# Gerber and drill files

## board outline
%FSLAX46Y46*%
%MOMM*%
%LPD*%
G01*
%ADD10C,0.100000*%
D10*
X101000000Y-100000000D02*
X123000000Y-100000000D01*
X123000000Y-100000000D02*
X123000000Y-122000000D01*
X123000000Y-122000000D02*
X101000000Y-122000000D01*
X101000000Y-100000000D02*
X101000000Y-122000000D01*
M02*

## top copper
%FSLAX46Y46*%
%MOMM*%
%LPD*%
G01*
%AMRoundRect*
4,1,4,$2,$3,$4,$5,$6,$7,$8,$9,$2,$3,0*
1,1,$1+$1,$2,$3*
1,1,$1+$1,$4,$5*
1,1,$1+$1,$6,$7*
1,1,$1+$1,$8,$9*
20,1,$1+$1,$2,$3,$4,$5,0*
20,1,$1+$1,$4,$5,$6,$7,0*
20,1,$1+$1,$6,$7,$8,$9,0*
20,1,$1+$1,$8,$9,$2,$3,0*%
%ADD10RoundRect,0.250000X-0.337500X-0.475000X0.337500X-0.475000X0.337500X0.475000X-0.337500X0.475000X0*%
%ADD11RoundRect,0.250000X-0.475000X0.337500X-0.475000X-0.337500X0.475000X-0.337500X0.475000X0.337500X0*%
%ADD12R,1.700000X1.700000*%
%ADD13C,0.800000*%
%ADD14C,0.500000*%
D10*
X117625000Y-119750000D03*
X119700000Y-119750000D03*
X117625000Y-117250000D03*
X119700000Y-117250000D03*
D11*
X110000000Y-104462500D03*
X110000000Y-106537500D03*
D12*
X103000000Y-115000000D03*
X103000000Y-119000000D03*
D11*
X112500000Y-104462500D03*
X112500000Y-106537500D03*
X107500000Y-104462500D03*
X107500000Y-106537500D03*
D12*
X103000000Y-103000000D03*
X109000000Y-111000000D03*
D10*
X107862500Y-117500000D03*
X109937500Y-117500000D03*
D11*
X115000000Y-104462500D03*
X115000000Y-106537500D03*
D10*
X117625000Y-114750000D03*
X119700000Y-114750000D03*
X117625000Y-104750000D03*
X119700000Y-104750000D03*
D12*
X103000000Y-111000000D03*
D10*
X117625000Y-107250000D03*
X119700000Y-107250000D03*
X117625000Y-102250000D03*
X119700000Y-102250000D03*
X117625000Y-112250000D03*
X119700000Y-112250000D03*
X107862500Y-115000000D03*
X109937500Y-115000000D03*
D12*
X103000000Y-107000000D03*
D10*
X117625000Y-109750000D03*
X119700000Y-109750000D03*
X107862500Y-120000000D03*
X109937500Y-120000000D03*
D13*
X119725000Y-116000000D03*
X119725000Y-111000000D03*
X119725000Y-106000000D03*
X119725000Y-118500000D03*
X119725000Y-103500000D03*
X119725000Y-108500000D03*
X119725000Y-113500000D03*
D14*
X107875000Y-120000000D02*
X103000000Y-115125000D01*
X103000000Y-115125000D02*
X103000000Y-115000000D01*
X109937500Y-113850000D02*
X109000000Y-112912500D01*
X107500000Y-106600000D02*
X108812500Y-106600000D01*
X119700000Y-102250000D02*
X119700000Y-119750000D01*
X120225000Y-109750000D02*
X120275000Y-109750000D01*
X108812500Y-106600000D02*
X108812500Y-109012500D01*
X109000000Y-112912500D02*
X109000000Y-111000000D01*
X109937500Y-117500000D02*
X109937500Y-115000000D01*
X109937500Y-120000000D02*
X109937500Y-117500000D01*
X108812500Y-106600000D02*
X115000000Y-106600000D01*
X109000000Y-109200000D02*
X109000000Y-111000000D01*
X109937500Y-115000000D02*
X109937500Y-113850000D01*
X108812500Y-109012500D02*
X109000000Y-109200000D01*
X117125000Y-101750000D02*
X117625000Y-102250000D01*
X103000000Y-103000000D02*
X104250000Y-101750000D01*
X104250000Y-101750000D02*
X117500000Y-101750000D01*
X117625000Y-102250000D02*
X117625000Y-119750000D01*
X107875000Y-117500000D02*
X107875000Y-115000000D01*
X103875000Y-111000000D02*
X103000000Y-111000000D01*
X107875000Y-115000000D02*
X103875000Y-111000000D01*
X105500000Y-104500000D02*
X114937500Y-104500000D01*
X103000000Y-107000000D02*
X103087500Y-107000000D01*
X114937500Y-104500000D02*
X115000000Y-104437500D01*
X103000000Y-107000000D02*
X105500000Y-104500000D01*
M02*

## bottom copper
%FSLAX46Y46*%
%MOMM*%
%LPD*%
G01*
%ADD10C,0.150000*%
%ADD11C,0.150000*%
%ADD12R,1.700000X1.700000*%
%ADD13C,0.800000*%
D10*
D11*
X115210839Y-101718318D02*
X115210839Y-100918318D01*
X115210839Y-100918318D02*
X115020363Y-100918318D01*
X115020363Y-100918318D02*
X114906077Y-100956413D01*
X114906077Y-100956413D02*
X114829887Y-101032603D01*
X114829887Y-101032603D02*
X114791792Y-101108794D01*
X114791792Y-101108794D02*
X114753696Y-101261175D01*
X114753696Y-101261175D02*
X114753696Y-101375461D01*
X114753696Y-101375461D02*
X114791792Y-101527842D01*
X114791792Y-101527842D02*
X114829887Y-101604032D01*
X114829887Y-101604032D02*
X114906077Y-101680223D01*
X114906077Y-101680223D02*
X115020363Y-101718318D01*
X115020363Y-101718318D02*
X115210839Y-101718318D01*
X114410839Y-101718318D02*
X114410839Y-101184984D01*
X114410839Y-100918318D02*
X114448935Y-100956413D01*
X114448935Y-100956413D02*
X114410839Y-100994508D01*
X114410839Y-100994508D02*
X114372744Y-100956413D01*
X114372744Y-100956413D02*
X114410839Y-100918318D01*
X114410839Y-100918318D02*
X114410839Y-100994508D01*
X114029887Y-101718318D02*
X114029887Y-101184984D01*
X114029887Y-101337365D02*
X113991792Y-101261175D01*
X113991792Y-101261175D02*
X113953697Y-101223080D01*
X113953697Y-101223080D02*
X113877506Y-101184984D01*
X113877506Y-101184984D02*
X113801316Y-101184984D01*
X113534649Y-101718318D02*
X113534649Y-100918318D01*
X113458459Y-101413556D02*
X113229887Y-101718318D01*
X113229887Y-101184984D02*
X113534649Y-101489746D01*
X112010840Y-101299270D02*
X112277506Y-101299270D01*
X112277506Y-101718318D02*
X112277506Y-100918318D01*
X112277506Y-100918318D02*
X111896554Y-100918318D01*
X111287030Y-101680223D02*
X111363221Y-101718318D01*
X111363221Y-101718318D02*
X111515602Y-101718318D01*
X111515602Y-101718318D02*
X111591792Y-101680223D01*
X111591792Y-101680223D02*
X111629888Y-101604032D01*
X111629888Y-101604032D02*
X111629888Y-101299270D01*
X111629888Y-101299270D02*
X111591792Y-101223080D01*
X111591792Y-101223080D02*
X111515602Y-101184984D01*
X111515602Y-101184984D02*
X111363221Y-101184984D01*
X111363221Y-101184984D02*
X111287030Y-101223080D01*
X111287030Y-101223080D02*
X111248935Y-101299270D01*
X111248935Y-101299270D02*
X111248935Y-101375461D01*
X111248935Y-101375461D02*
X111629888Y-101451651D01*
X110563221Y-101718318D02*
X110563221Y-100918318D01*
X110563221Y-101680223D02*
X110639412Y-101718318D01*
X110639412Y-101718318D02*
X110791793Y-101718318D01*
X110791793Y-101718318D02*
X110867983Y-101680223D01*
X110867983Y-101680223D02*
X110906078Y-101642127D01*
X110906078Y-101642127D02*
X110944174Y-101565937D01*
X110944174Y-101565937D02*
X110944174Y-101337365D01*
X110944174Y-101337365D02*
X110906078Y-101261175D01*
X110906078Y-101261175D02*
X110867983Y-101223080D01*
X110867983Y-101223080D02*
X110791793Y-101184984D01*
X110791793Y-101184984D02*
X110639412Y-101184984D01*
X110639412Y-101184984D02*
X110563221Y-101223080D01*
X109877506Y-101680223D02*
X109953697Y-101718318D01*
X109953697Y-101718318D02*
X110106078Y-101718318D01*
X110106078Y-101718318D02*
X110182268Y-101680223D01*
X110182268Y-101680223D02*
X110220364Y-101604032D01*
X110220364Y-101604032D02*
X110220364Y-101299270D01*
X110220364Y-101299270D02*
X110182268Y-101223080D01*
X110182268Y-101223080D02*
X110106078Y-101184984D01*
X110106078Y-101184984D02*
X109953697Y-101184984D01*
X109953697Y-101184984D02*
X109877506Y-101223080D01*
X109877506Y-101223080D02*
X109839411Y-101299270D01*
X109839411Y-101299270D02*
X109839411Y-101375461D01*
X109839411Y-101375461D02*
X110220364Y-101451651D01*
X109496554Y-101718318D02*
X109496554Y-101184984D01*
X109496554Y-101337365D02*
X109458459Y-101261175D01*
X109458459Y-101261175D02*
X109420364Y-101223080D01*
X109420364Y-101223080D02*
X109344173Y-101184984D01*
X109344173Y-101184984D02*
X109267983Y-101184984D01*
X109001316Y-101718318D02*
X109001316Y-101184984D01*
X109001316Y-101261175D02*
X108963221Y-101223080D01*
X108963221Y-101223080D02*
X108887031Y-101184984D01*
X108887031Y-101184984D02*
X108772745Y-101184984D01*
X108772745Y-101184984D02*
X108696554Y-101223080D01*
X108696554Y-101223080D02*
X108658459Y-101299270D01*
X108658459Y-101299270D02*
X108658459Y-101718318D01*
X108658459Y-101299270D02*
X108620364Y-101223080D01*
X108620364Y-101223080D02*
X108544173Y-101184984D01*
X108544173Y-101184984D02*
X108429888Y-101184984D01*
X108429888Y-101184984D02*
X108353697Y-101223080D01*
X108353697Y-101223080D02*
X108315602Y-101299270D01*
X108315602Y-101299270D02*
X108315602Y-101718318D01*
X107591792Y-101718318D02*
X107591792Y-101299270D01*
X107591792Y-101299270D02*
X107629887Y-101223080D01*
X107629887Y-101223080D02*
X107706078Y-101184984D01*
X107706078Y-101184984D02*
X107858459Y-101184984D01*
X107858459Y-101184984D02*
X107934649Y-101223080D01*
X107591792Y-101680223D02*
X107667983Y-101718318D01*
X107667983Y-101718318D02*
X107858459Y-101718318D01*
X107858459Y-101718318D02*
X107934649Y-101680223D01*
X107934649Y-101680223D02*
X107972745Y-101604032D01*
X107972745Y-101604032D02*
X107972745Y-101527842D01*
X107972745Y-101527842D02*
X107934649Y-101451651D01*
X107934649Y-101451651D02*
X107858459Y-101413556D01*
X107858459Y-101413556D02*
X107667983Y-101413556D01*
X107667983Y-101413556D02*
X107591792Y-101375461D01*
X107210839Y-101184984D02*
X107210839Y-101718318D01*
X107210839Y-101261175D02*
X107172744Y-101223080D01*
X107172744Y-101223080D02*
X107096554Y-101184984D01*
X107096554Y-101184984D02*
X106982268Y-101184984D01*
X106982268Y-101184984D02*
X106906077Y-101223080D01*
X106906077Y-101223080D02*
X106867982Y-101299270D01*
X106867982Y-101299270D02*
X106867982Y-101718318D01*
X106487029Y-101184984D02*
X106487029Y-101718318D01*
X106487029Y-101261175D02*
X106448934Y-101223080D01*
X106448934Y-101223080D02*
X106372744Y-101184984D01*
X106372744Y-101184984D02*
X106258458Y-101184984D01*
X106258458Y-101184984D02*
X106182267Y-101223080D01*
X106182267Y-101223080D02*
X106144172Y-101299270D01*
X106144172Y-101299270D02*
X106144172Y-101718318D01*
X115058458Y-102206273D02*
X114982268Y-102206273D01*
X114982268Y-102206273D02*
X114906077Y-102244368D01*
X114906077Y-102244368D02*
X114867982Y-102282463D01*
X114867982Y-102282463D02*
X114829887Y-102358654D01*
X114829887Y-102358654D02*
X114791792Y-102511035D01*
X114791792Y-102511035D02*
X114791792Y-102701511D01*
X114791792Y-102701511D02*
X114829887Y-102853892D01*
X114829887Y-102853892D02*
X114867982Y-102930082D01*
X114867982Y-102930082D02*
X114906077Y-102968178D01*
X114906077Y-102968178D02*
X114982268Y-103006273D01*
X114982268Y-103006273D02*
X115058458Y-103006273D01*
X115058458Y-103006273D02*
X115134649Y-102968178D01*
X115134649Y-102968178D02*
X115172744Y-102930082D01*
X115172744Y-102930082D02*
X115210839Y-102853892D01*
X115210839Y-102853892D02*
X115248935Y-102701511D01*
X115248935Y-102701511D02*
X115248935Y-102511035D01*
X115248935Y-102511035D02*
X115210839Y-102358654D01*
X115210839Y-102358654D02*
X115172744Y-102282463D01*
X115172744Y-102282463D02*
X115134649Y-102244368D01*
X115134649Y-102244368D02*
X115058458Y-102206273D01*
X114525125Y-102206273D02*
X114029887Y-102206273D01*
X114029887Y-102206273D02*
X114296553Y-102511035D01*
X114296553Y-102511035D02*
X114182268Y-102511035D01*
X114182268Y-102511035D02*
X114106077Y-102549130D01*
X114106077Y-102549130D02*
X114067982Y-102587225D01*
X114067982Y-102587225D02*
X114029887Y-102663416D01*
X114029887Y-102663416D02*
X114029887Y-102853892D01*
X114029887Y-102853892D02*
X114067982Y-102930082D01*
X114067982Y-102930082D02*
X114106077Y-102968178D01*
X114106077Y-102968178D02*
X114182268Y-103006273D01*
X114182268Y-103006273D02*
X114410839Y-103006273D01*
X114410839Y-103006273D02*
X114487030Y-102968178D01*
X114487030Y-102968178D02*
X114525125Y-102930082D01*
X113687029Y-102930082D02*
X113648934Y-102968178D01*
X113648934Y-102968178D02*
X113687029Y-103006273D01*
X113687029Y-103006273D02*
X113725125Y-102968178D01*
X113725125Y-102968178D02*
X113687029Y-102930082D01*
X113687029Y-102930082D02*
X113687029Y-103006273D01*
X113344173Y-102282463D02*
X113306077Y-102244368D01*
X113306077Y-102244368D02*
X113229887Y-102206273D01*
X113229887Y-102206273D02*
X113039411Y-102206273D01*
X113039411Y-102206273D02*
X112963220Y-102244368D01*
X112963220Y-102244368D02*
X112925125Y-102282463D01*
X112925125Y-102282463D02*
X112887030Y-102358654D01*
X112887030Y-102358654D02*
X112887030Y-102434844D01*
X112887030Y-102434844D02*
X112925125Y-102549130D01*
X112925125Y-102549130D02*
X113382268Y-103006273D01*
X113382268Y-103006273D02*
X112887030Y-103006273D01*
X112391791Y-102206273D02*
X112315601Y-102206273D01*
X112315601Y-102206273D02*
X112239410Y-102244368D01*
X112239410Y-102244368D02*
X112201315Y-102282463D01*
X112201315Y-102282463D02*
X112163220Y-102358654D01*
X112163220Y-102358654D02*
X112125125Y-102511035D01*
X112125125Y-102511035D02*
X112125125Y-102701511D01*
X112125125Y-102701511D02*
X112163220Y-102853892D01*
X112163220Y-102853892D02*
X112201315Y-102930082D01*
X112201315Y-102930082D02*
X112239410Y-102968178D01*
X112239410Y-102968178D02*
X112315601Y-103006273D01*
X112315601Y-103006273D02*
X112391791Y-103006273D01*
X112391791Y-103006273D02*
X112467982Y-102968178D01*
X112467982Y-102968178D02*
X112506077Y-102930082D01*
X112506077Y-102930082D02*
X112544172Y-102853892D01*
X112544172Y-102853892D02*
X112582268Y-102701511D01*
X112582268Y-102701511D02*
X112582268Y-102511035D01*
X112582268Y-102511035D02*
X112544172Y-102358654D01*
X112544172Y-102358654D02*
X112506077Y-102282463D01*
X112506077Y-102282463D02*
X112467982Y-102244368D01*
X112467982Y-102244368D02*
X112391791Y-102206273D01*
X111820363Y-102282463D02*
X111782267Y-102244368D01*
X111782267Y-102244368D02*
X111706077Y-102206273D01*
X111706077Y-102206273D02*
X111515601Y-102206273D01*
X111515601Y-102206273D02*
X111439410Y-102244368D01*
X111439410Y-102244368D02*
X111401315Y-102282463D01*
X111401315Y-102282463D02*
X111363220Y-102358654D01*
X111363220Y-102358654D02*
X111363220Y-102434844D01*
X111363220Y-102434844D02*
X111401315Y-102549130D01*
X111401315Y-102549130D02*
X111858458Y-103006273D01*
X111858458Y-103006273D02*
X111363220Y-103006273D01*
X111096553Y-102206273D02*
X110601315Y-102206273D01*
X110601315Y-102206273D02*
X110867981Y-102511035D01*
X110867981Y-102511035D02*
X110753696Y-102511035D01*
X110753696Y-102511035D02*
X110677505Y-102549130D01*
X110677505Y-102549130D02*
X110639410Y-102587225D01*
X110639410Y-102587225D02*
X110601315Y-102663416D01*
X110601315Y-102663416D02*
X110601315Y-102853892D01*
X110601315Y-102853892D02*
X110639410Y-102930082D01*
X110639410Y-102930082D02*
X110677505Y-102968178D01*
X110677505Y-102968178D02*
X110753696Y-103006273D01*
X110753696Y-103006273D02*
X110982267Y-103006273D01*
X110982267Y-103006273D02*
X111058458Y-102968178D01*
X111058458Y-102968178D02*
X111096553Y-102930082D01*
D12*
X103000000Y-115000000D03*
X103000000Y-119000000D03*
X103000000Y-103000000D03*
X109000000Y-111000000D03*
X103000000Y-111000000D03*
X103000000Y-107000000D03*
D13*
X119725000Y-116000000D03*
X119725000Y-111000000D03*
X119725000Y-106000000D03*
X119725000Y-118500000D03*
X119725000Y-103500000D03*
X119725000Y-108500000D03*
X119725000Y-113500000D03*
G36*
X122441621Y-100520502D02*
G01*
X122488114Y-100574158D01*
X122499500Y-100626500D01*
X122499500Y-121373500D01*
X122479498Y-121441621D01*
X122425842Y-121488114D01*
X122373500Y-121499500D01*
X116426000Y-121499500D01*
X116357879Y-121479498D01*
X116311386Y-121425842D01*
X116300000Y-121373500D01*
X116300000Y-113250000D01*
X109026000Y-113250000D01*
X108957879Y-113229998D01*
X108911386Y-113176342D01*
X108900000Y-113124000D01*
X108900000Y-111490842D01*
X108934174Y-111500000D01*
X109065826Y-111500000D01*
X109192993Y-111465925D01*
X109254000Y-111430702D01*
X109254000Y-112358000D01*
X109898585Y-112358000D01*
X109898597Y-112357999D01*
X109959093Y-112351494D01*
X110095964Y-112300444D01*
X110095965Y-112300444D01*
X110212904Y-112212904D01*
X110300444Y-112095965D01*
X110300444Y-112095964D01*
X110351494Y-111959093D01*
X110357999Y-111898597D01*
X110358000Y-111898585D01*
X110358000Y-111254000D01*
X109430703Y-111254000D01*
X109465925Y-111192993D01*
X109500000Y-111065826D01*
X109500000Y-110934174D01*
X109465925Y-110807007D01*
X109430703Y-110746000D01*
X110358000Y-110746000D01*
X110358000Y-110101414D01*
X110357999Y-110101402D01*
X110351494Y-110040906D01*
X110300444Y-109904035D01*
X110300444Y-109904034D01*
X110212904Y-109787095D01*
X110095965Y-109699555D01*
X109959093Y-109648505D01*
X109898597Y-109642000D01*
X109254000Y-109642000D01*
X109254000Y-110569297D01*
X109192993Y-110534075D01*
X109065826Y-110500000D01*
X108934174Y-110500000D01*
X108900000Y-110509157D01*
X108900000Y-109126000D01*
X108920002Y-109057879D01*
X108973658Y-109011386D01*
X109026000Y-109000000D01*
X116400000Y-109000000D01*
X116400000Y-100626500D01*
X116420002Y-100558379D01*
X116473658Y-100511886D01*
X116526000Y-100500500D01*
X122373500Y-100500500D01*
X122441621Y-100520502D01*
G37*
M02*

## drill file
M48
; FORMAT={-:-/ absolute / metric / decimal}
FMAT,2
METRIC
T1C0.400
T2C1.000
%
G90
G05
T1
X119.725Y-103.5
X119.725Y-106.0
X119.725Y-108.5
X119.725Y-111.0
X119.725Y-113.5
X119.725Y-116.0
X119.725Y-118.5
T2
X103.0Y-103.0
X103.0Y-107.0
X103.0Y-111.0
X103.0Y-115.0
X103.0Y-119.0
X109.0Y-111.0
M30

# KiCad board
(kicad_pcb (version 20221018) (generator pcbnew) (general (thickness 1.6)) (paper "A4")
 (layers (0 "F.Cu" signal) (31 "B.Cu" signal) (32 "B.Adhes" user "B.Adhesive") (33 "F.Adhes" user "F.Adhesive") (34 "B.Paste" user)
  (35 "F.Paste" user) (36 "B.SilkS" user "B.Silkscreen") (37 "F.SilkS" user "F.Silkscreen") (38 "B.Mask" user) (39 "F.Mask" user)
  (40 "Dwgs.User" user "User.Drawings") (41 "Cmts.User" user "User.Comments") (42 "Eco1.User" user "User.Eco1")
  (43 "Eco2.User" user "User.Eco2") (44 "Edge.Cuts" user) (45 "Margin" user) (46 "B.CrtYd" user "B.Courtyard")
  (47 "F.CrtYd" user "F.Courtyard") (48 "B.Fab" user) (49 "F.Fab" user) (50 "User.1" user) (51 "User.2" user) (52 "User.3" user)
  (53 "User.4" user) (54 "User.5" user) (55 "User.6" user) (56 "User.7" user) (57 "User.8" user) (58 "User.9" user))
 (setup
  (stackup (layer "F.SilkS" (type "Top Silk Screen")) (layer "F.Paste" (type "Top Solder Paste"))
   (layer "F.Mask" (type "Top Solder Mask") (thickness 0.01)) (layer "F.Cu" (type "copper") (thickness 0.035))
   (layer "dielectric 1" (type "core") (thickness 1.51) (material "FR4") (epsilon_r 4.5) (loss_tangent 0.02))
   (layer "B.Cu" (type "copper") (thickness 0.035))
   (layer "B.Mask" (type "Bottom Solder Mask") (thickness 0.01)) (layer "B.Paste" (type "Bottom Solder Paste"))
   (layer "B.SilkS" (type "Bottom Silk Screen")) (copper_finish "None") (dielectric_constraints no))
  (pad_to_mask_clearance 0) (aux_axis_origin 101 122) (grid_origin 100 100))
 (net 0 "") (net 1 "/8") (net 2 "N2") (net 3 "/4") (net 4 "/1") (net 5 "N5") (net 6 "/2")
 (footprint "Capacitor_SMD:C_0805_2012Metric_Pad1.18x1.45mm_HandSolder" (layer "F.Cu") (at 118.6625 119.75)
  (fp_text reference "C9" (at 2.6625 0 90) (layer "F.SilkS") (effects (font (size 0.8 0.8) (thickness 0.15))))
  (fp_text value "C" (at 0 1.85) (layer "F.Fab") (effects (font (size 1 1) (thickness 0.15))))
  (pad "1" smd roundrect (at -1.0375 0) (size 1.175 1.45) (layers "F.Cu" "F.Paste" "F.Mask") (roundrect_rratio 0.2127659574) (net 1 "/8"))
  (pad "2" smd roundrect (at 1.0375 0) (size 1.175 1.45) (layers "F.Cu" "F.Paste" "F.Mask") (roundrect_rratio 0.2127659574) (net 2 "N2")))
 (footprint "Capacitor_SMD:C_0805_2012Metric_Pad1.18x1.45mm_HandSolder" (layer "F.Cu") (at 118.6625 117.25)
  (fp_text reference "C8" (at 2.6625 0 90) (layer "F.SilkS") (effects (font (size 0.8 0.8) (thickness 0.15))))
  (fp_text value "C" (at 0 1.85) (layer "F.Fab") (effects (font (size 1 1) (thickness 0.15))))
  (pad "1" smd roundrect (at -1.0375 0) (size 1.175 1.45) (layers "F.Cu" "F.Paste" "F.Mask") (roundrect_rratio 0.2127659574) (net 1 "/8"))
  (pad "2" smd roundrect (at 1.0375 0) (size 1.175 1.45) (layers "F.Cu" "F.Paste" "F.Mask") (roundrect_rratio 0.2127659574) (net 2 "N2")))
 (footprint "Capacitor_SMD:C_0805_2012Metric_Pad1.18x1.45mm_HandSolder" (layer "F.Cu") (at 110 105.5 -90)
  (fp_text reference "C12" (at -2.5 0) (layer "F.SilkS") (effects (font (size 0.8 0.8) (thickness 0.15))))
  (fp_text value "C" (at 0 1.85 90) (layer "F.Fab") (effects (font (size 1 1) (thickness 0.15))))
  (pad "1" smd roundrect (at -1.0375 0 270) (size 1.175 1.45) (layers "F.Cu" "F.Paste" "F.Mask") (roundrect_rratio 0.2127659574)
   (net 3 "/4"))
  (pad "2" smd roundrect (at 1.0375 0 270) (size 1.175 1.45) (layers "F.Cu" "F.Paste" "F.Mask") (roundrect_rratio 0.2127659574) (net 2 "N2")))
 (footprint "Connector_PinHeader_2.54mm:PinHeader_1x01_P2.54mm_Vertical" (layer "F.Cu") (at 103 115)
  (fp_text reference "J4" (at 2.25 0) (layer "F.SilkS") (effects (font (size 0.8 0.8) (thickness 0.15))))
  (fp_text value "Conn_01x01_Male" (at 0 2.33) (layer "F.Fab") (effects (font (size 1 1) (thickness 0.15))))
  (pad "1" thru_hole rect (at 0 0) (size 1.7 1.7) (drill 1) (layers "*.Cu" "*.Mask") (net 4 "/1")))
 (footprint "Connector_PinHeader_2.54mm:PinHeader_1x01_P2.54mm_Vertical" (layer "F.Cu") (at 103 119)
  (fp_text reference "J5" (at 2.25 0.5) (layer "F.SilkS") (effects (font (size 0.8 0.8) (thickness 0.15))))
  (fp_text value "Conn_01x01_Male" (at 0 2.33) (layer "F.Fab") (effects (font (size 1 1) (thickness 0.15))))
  (pad "1" thru_hole rect (at 0 0) (size 1.7 1.7) (drill 1) (layers "*.Cu" "*.Mask") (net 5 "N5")))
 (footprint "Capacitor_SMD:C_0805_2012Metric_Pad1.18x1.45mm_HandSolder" (layer "F.Cu") (at 112.5 105.5 -90)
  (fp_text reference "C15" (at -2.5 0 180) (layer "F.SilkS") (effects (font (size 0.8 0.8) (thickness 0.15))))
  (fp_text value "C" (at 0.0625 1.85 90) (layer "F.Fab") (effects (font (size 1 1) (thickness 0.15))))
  (pad "1" smd roundrect (at -1.0375 0 270) (size 1.175 1.45) (layers "F.Cu" "F.Paste" "F.Mask") (roundrect_rratio 0.2127659574)
   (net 3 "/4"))
  (pad "2" smd roundrect (at 1.0375 0 270) (size 1.175 1.45) (layers "F.Cu" "F.Paste" "F.Mask") (roundrect_rratio 0.2127659574) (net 2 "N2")))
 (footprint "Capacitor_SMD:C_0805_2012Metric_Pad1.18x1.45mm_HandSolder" (layer "F.Cu") (at 107.5 105.5 -90)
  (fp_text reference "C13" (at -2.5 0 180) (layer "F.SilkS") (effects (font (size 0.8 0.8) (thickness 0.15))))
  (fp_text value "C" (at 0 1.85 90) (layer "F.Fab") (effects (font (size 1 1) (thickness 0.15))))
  (pad "1" smd roundrect (at -1.0375 0 270) (size 1.175 1.45) (layers "F.Cu" "F.Paste" "F.Mask") (roundrect_rratio 0.2127659574)
   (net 3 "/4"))
  (pad "2" smd roundrect (at 1.0375 0 270) (size 1.175 1.45) (layers "F.Cu" "F.Paste" "F.Mask") (roundrect_rratio 0.2127659574) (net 2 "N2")))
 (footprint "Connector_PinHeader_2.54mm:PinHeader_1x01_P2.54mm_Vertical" (layer "F.Cu") (at 103 103)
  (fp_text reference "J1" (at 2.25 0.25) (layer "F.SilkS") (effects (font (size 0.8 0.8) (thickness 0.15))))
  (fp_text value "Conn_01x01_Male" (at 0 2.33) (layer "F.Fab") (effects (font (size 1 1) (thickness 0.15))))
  (pad "1" thru_hole rect (at 0 0) (size 1.7 1.7) (drill 1) (layers "*.Cu" "*.Mask") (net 1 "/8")))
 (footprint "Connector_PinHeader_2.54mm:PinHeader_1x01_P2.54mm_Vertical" (layer "F.Cu") (at 109 111)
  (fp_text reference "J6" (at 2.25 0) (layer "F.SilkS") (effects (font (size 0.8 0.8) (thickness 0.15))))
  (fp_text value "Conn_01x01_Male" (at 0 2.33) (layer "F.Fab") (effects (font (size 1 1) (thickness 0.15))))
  (pad "1" thru_hole rect (at 0 0) (size 1.7 1.7) (drill 1) (layers "*.Cu" "*.Mask") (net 2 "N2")))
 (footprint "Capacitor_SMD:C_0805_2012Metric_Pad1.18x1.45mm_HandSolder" (layer "F.Cu") (at 108.9 117.5)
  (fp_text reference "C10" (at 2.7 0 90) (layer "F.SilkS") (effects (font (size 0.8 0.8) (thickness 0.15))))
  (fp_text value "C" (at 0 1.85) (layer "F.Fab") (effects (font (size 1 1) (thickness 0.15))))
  (pad "1" smd roundrect (at -1.0375 0) (size 1.175 1.45) (layers "F.Cu" "F.Paste" "F.Mask") (roundrect_rratio 0.2127659574) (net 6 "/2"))
  (pad "2" smd roundrect (at 1.0375 0) (size 1.175 1.45) (layers "F.Cu" "F.Paste" "F.Mask") (roundrect_rratio 0.2127659574) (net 2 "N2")))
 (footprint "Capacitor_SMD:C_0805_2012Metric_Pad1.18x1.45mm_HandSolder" (layer "F.Cu") (at 115 105.5 -90)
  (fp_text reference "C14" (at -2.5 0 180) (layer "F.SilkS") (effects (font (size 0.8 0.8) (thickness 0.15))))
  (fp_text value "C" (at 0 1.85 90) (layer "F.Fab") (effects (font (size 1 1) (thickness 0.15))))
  (pad "1" smd roundrect (at -1.0375 0 270) (size 1.175 1.45) (layers "F.Cu" "F.Paste" "F.Mask") (roundrect_rratio 0.2127659574)
   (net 3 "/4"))
  (pad "2" smd roundrect (at 1.0375 0 270) (size 1.175 1.45) (layers "F.Cu" "F.Paste" "F.Mask") (roundrect_rratio 0.2127659574) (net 2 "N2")))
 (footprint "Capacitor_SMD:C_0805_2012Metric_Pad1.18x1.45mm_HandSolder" (layer "F.Cu") (at 118.6625 114.75)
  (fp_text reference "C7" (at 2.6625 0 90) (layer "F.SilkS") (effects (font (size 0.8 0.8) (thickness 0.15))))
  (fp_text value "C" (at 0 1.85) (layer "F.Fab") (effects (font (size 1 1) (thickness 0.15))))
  (pad "1" smd roundrect (at -1.0375 0) (size 1.175 1.45) (layers "F.Cu" "F.Paste" "F.Mask") (roundrect_rratio 0.2127659574) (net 1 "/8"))
  (pad "2" smd roundrect (at 1.0375 0) (size 1.175 1.45) (layers "F.Cu" "F.Paste" "F.Mask") (roundrect_rratio 0.2127659574) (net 2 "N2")))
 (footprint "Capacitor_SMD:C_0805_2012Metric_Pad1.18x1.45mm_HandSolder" (layer "F.Cu") (at 118.6625 104.75)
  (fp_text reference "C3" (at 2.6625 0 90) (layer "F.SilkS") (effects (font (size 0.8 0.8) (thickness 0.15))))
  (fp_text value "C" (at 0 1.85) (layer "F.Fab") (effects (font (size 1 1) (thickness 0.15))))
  (pad "1" smd roundrect (at -1.0375 0) (size 1.175 1.45) (layers "F.Cu" "F.Paste" "F.Mask") (roundrect_rratio 0.2127659574) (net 1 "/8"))
  (pad "2" smd roundrect (at 1.0375 0) (size 1.175 1.45) (layers "F.Cu" "F.Paste" "F.Mask") (roundrect_rratio 0.2127659574) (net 2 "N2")))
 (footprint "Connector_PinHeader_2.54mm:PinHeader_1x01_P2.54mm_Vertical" (layer "F.Cu") (at 103 111)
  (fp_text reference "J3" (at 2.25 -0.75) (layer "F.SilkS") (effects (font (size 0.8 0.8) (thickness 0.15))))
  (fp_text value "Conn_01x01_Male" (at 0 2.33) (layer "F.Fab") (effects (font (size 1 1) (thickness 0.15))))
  (pad "1" thru_hole rect (at 0 0) (size 1.7 1.7) (drill 1) (layers "*.Cu" "*.Mask") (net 6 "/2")))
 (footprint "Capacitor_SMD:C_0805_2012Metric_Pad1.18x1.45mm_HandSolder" (layer "F.Cu") (at 118.6625 107.25)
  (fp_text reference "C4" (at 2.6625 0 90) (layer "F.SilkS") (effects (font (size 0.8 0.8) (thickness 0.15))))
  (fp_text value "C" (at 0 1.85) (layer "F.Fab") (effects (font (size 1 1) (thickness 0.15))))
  (pad "1" smd roundrect (at -1.0375 0) (size 1.175 1.45) (layers "F.Cu" "F.Paste" "F.Mask") (roundrect_rratio 0.2127659574) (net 1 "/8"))
  (pad "2" smd roundrect (at 1.0375 0) (size 1.175 1.45) (layers "F.Cu" "F.Paste" "F.Mask") (roundrect_rratio 0.2127659574) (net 2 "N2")))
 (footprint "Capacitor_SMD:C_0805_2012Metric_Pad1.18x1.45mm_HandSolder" (layer "F.Cu") (at 118.6625 102.25)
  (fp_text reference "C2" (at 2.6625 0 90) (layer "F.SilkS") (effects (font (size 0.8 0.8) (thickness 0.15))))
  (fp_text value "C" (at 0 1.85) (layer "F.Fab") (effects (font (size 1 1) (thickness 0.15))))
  (pad "1" smd roundrect (at -1.0375 0) (size 1.175 1.45) (layers "F.Cu" "F.Paste" "F.Mask") (roundrect_rratio 0.2127659574) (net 1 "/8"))
  (pad "2" smd roundrect (at 1.0375 0) (size 1.175 1.45) (layers "F.Cu" "F.Paste" "F.Mask") (roundrect_rratio 0.2127659574) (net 2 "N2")))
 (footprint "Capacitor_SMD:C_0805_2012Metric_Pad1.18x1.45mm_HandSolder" (layer "F.Cu") (at 118.6625 112.25)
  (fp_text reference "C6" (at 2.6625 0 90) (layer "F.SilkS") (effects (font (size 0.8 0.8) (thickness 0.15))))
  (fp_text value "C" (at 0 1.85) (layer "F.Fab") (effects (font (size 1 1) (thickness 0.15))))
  (pad "1" smd roundrect (at -1.0375 0) (size 1.175 1.45) (layers "F.Cu" "F.Paste" "F.Mask") (roundrect_rratio 0.2127659574) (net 1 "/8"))
  (pad "2" smd roundrect (at 1.0375 0) (size 1.175 1.45) (layers "F.Cu" "F.Paste" "F.Mask") (roundrect_rratio 0.2127659574) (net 2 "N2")))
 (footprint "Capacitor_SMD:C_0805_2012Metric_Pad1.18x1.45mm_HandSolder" (layer "F.Cu") (at 108.9 115)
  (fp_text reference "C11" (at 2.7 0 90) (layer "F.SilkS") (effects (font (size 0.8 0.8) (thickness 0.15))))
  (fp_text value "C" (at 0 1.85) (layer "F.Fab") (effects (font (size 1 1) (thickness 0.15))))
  (pad "1" smd roundrect (at -1.0375 0) (size 1.175 1.45) (layers "F.Cu" "F.Paste" "F.Mask") (roundrect_rratio 0.2127659574) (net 6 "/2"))
  (pad "2" smd roundrect (at 1.0375 0) (size 1.175 1.45) (layers "F.Cu" "F.Paste" "F.Mask") (roundrect_rratio 0.2127659574) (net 2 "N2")))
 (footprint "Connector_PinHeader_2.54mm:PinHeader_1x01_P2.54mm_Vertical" (layer "F.Cu") (at 103 107)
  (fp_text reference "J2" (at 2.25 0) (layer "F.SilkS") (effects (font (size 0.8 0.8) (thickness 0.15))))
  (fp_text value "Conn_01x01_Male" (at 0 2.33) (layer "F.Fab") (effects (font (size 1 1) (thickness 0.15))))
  (pad "1" thru_hole rect (at 0 0) (size 1.7 1.7) (drill 1) (layers "*.Cu" "*.Mask") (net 3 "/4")))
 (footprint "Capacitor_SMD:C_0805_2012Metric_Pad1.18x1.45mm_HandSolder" (layer "F.Cu") (at 118.6625 109.75)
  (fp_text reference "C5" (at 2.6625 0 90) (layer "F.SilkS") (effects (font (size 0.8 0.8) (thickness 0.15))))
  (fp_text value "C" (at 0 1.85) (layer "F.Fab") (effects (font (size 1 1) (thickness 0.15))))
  (pad "1" smd roundrect (at -1.0375 0) (size 1.175 1.45) (layers "F.Cu" "F.Paste" "F.Mask") (roundrect_rratio 0.2127659574) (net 1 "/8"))
  (pad "2" smd roundrect (at 1.0375 0) (size 1.175 1.45) (layers "F.Cu" "F.Paste" "F.Mask") (roundrect_rratio 0.2127659574) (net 2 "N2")))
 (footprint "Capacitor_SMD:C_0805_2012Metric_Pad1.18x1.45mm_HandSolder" (layer "F.Cu") (at 108.9 120)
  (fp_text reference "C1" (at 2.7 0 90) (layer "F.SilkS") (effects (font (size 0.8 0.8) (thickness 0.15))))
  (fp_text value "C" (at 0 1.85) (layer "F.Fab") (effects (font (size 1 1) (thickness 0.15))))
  (pad "1" smd roundrect (at -1.0375 0) (size 1.175 1.45) (layers "F.Cu" "F.Paste" "F.Mask") (roundrect_rratio 0.2127659574) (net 4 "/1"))
  (pad "2" smd roundrect (at 1.0375 0) (size 1.175 1.45) (layers "F.Cu" "F.Paste" "F.Mask") (roundrect_rratio 0.2127659574) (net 2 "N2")))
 (gr_line (start 101 100) (end 123 100) (stroke (width 0.1) (type solid)) (layer "Edge.Cuts"))
 (gr_line (start 123 100) (end 123 122) (stroke (width 0.1) (type solid)) (layer "Edge.Cuts"))
 (gr_line (start 123 122) (end 101 122) (stroke (width 0.1) (type solid)) (layer "Edge.Cuts"))
 (gr_line (start 101 100) (end 101 122) (stroke (width 0.1) (type solid)) (layer "Edge.Cuts"))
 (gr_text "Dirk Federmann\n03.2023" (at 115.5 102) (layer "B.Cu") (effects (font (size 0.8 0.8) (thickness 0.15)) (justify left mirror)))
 (segment (start 107.875 120) (end 103 115.125) (width 0.5) (layer "F.Cu") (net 4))
 (segment (start 103 115.125) (end 103 115) (width 0.5) (layer "F.Cu") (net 4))
 (segment (start 109.9375 113.85) (end 109 112.9125) (width 0.5) (layer "F.Cu") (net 2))
 (segment (start 107.5 106.6) (end 108.8125 106.6) (width 0.5) (layer "F.Cu") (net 2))
 (segment (start 119.7 102.25) (end 119.7 119.75) (width 0.5) (layer "F.Cu") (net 2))
 (segment (start 120.225 109.75) (end 120.275 109.75) (width 0.5) (layer "F.Cu") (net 2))
 (segment (start 108.8125 106.6) (end 108.8125 109.0125) (width 0.5) (layer "F.Cu") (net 2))
 (segment (start 109 112.9125) (end 109 111) (width 0.5) (layer "F.Cu") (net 2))
 (segment (start 109.9375 117.5) (end 109.9375 115) (width 0.5) (layer "F.Cu") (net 2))
 (segment (start 109.9375 120) (end 109.9375 117.5) (width 0.5) (layer "F.Cu") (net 2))
 (segment (start 108.8125 106.6) (end 115 106.6) (width 0.5) (layer "F.Cu") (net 2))
 (segment (start 109 109.2) (end 109 111) (width 0.5) (layer "F.Cu") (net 2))
 (segment (start 109.9375 115) (end 109.9375 113.85) (width 0.5) (layer "F.Cu") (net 2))
 (segment (start 108.8125 109.0125) (end 109 109.2) (width 0.5) (layer "F.Cu") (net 2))
 (via (at 119.725 116) (size 0.8) (drill 0.4) (layers "F.Cu" "B.Cu") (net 2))
 (via (at 119.725 111) (size 0.8) (drill 0.4) (layers "F.Cu" "B.Cu") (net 2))
 (via (at 119.725 106) (size 0.8) (drill 0.4) (layers "F.Cu" "B.Cu") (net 2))
 (via (at 119.725 118.5) (size 0.8) (drill 0.4) (layers "F.Cu" "B.Cu") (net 2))
 (via (at 119.725 103.5) (size 0.8) (drill 0.4) (layers "F.Cu" "B.Cu") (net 2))
 (via (at 119.725 108.5) (size 0.8) (drill 0.4) (layers "F.Cu" "B.Cu") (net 2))
 (via (at 119.725 113.5) (size 0.8) (drill 0.4) (layers "F.Cu" "B.Cu") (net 2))
 (segment (start 117.125 101.75) (end 117.625 102.25) (width 0.5) (layer "F.Cu") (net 1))
 (segment (start 103 103) (end 104.25 101.75) (width 0.5) (layer "F.Cu") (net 1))
 (segment (start 104.25 101.75) (end 117.5 101.75) (width 0.5) (layer "F.Cu") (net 1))
 (segment (start 117.625 102.25) (end 117.625 119.75) (width 0.5) (layer "F.Cu") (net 1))
 (segment (start 107.875 117.5) (end 107.875 115) (width 0.5) (layer "F.Cu") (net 6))
 (segment (start 103.875 111) (end 103 111) (width 0.5) (layer "F.Cu") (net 6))
 (segment (start 107.875 115) (end 103.875 111) (width 0.5) (layer "F.Cu") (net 6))
 (segment (start 105.5 104.5) (end 114.9375 104.5) (width 0.5) (layer "F.Cu") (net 3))
 (segment (start 103 107) (end 103.0875 107) (width 0.5) (layer "F.Cu") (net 3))
 (segment (start 114.9375 104.5) (end 115 104.4375) (width 0.5) (layer "F.Cu") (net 3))
 (segment (start 103 107) (end 105.5 104.5) (width 0.5) (layer "F.Cu") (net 3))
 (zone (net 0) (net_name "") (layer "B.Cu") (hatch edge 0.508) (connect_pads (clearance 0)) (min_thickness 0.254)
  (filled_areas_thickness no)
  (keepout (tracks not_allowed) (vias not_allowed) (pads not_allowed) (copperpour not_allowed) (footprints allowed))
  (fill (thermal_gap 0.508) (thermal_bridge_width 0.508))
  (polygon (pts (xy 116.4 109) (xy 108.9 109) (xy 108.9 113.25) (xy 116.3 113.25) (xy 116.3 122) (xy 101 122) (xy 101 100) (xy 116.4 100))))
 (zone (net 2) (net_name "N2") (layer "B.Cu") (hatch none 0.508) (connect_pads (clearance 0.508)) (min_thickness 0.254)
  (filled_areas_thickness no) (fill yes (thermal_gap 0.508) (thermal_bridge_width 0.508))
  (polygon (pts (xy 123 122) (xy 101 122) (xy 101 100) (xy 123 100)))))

